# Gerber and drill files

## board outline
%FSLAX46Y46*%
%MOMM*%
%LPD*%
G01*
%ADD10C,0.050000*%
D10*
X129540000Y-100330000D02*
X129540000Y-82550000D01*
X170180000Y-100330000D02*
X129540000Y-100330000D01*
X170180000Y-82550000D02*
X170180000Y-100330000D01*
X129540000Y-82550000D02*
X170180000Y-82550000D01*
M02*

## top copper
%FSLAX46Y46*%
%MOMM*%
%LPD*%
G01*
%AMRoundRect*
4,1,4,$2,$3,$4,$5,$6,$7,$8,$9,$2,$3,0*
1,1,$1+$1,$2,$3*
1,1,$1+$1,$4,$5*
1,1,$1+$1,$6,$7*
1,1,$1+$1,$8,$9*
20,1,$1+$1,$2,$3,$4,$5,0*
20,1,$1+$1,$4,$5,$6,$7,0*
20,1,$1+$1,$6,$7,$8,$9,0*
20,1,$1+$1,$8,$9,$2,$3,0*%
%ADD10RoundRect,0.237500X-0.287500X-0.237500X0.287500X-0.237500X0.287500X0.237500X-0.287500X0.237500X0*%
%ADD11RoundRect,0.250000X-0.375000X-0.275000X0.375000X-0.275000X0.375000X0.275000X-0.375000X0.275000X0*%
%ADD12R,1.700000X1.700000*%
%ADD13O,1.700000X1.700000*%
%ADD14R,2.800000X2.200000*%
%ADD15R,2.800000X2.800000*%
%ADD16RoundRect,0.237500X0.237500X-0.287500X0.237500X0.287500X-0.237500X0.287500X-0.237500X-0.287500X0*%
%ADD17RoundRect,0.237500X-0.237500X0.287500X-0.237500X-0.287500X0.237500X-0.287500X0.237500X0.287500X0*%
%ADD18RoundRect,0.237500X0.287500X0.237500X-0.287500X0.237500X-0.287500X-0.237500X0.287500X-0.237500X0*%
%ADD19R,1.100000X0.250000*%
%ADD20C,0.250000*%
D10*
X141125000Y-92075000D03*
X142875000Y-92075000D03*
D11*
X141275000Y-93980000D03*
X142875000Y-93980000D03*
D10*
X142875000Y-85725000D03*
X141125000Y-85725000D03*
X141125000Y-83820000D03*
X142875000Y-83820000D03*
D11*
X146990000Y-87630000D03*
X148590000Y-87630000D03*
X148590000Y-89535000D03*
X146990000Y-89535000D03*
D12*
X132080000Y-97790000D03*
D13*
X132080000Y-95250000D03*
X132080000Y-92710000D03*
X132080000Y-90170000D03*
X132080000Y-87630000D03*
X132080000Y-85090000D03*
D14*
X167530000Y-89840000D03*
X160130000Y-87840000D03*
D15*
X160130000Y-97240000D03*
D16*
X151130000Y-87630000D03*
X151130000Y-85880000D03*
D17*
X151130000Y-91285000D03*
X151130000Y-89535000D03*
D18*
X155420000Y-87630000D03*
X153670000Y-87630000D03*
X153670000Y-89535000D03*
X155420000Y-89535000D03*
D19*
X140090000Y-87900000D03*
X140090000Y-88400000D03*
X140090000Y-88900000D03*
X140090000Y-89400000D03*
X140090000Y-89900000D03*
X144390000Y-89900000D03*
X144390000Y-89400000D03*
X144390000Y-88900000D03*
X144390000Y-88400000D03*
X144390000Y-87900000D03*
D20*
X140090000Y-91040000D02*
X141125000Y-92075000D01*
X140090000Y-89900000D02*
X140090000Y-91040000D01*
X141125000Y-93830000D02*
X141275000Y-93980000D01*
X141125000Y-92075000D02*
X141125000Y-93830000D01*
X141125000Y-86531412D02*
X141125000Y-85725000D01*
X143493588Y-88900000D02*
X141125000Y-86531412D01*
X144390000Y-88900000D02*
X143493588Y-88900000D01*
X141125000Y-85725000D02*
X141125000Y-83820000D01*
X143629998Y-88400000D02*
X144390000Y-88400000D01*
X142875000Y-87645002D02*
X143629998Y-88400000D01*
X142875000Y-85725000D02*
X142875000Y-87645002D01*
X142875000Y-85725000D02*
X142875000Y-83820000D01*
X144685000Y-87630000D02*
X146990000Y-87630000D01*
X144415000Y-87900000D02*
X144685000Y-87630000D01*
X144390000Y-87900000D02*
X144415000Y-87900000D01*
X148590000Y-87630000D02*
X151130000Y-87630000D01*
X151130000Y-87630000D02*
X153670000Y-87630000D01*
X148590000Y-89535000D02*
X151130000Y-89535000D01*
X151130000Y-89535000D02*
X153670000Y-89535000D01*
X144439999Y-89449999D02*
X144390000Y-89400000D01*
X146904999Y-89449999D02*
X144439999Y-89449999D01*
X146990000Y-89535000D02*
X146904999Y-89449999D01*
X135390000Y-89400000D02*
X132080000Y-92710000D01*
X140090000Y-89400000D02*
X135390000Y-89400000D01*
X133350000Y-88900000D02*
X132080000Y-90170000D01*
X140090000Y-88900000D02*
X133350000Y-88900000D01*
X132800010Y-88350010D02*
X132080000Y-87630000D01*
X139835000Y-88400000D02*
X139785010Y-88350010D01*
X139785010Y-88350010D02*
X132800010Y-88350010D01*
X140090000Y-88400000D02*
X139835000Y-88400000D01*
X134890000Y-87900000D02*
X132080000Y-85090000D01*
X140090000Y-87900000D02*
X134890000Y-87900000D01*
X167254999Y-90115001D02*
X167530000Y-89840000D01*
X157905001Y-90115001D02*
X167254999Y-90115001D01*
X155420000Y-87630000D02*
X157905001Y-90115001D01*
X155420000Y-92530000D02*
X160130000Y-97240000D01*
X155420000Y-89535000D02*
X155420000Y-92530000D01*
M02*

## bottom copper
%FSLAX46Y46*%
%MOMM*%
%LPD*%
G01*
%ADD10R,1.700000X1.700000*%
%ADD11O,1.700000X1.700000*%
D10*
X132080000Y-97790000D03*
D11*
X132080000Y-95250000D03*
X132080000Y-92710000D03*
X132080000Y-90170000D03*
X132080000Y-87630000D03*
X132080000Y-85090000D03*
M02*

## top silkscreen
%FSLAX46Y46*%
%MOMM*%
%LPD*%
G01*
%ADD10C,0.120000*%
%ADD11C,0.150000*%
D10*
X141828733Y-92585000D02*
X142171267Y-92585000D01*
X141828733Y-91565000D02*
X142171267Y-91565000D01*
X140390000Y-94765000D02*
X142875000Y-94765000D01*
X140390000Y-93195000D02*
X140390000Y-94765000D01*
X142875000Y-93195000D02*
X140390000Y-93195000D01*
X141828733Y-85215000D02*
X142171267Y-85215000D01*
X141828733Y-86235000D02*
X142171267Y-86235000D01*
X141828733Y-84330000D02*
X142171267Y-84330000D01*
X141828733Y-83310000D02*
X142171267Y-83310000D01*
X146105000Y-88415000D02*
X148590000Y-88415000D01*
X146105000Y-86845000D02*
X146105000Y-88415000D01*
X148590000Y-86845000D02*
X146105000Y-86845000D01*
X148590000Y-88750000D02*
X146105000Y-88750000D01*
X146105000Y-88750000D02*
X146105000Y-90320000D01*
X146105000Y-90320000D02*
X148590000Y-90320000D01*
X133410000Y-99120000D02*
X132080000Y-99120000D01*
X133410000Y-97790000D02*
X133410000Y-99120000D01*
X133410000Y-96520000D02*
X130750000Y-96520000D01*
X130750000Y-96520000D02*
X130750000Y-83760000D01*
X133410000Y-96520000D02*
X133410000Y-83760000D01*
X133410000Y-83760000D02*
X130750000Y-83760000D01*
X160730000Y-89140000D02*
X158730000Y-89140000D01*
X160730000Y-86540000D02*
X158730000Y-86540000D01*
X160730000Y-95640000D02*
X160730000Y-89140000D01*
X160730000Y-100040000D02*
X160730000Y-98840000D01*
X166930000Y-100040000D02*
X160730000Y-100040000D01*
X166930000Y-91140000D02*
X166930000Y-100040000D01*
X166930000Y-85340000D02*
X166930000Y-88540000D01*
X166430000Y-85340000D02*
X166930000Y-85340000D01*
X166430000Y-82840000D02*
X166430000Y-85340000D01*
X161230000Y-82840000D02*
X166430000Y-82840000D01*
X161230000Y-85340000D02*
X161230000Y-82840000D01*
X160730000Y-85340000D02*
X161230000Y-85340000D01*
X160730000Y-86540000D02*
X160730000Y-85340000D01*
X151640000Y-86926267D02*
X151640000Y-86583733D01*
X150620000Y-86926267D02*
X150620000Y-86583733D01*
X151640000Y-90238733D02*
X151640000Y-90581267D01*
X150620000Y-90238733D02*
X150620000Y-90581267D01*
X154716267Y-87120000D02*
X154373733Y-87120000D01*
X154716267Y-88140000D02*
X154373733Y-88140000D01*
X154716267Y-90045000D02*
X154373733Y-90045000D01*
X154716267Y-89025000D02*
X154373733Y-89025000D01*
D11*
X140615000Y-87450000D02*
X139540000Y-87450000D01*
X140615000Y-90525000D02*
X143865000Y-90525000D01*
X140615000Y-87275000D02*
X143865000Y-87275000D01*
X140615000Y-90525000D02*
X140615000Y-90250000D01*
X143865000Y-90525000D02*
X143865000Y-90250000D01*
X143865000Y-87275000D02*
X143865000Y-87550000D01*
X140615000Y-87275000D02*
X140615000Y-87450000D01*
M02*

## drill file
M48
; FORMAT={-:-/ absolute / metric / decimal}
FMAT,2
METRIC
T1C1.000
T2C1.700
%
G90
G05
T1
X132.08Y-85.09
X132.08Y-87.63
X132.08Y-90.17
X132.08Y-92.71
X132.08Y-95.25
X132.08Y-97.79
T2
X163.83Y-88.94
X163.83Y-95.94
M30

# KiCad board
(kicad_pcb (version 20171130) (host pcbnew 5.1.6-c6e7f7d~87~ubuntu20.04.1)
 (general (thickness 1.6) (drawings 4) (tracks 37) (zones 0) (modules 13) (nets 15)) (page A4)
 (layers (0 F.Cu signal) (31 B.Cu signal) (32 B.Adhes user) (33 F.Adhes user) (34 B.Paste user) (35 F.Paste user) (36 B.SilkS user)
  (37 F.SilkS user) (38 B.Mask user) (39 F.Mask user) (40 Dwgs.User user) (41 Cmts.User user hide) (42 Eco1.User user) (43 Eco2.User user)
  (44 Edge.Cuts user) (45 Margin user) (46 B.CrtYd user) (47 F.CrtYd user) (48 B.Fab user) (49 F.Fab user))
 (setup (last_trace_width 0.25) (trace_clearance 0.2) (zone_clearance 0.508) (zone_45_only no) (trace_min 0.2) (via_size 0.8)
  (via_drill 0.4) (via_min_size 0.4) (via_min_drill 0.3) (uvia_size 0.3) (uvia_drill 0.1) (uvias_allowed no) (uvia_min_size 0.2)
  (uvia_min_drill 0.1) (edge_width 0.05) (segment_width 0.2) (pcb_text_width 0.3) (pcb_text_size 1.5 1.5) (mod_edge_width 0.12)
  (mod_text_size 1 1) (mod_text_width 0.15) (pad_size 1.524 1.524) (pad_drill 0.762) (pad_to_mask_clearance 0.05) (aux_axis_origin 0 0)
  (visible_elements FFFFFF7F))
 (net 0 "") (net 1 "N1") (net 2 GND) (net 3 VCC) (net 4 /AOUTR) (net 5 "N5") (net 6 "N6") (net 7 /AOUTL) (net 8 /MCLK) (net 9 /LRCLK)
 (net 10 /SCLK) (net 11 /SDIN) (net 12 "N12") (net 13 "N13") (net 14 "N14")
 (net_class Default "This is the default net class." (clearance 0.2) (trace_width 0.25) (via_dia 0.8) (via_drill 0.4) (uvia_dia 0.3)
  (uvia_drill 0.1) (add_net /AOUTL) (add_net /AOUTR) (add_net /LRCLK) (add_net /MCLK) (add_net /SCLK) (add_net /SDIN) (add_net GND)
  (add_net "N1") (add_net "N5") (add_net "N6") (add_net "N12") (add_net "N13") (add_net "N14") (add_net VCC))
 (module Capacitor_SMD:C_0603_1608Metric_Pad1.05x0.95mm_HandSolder (layer F.Cu) (at 142 92.075)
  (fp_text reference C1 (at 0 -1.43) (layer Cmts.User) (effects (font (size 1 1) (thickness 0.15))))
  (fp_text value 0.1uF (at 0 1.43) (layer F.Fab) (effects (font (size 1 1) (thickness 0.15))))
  (fp_line (start -0.171267 0.51) (end 0.171267 0.51) (layer F.SilkS) (width 0.12))
  (fp_line (start -0.171267 -0.51) (end 0.171267 -0.51) (layer F.SilkS) (width 0.12))
  (pad 1 smd roundrect (at -0.875 0) (size 1.05 0.95) (layers F.Cu F.Paste F.Mask) (roundrect_rratio 0.25) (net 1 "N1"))
  (pad 2 smd roundrect (at 0.875 0) (size 1.05 0.95) (layers F.Cu F.Paste F.Mask) (roundrect_rratio 0.25) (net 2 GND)))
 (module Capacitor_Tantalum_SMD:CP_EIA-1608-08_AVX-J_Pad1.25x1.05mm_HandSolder (layer F.Cu) (at 142.075 93.98)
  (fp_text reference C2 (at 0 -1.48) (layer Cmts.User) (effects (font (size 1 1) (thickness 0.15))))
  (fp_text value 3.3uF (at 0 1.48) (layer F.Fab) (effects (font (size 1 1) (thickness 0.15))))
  (fp_line (start -1.685 0.785) (end 0.8 0.785) (layer F.SilkS) (width 0.12))
  (fp_line (start -1.685 -0.785) (end -1.685 0.785) (layer F.SilkS) (width 0.12))
  (fp_line (start 0.8 -0.785) (end -1.685 -0.785) (layer F.SilkS) (width 0.12))
  (pad 1 smd roundrect (at -0.8 0) (size 1.25 1.05) (layers F.Cu F.Paste F.Mask) (roundrect_rratio 0.238095) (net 1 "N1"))
  (pad 2 smd roundrect (at 0.8 0) (size 1.25 1.05) (layers F.Cu F.Paste F.Mask) (roundrect_rratio 0.238095) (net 2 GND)))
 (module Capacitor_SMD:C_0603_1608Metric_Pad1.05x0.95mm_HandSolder (layer F.Cu) (at 142 85.725)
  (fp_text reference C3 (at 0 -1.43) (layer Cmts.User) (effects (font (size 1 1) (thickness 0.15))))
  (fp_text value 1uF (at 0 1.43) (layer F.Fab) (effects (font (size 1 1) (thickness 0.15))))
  (fp_line (start -0.171267 -0.51) (end 0.171267 -0.51) (layer F.SilkS) (width 0.12))
  (fp_line (start -0.171267 0.51) (end 0.171267 0.51) (layer F.SilkS) (width 0.12))
  (pad 2 smd roundrect (at 0.875 0) (size 1.05 0.95) (layers F.Cu F.Paste F.Mask) (roundrect_rratio 0.25) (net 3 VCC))
  (pad 1 smd roundrect (at -0.875 0) (size 1.05 0.95) (layers F.Cu F.Paste F.Mask) (roundrect_rratio 0.25) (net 2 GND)))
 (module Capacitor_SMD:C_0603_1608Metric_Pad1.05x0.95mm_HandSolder (layer F.Cu) (at 142 83.82)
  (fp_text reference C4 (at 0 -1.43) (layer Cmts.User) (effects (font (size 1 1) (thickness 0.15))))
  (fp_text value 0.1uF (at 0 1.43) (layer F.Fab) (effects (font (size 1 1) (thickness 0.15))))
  (fp_line (start -0.171267 0.51) (end 0.171267 0.51) (layer F.SilkS) (width 0.12))
  (fp_line (start -0.171267 -0.51) (end 0.171267 -0.51) (layer F.SilkS) (width 0.12))
  (pad 1 smd roundrect (at -0.875 0) (size 1.05 0.95) (layers F.Cu F.Paste F.Mask) (roundrect_rratio 0.25) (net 2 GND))
  (pad 2 smd roundrect (at 0.875 0) (size 1.05 0.95) (layers F.Cu F.Paste F.Mask) (roundrect_rratio 0.25) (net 3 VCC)))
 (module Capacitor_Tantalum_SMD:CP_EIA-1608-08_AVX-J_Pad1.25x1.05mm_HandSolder (layer F.Cu) (at 147.79 87.63)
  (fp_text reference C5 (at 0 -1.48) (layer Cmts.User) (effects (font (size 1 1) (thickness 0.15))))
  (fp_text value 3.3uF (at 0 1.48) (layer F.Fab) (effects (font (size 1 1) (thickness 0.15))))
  (fp_line (start -1.685 0.785) (end 0.8 0.785) (layer F.SilkS) (width 0.12))
  (fp_line (start -1.685 -0.785) (end -1.685 0.785) (layer F.SilkS) (width 0.12))
  (fp_line (start 0.8 -0.785) (end -1.685 -0.785) (layer F.SilkS) (width 0.12))
  (pad 1 smd roundrect (at -0.8 0) (size 1.25 1.05) (layers F.Cu F.Paste F.Mask) (roundrect_rratio 0.238095) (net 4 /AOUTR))
  (pad 2 smd roundrect (at 0.8 0) (size 1.25 1.05) (layers F.Cu F.Paste F.Mask) (roundrect_rratio 0.238095) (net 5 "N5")))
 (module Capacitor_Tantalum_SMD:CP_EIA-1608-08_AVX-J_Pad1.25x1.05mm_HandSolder (layer F.Cu) (at 147.79 89.535)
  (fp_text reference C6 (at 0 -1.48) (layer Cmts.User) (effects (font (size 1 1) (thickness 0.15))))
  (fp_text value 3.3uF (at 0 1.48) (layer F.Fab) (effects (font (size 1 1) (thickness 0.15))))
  (fp_line (start 0.8 -0.785) (end -1.685 -0.785) (layer F.SilkS) (width 0.12))
  (fp_line (start -1.685 -0.785) (end -1.685 0.785) (layer F.SilkS) (width 0.12))
  (fp_line (start -1.685 0.785) (end 0.8 0.785) (layer F.SilkS) (width 0.12))
  (pad 2 smd roundrect (at 0.8 0) (size 1.25 1.05) (layers F.Cu F.Paste F.Mask) (roundrect_rratio 0.238095) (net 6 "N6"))
  (pad 1 smd roundrect (at -0.8 0) (size 1.25 1.05) (layers F.Cu F.Paste F.Mask) (roundrect_rratio 0.238095) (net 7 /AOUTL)))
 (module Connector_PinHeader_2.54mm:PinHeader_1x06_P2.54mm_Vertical (layer F.Cu) (at 132.08 97.79 180)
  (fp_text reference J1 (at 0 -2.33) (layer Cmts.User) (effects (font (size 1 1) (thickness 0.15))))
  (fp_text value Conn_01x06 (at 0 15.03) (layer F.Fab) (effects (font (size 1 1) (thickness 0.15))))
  (fp_line (start -1.33 -1.33) (end 0 -1.33) (layer F.SilkS) (width 0.12))
  (fp_line (start -1.33 0) (end -1.33 -1.33) (layer F.SilkS) (width 0.12))
  (fp_line (start -1.33 1.27) (end 1.33 1.27) (layer F.SilkS) (width 0.12))
  (fp_line (start 1.33 1.27) (end 1.33 14.03) (layer F.SilkS) (width 0.12))
  (fp_line (start -1.33 1.27) (end -1.33 14.03) (layer F.SilkS) (width 0.12))
  (fp_line (start -1.33 14.03) (end 1.33 14.03) (layer F.SilkS) (width 0.12))
  (pad 1 thru_hole rect (at 0 0 180) (size 1.7 1.7) (drill 1) (layers *.Cu *.Mask) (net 3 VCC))
  (pad 2 thru_hole oval (at 0 2.54 180) (size 1.7 1.7) (drill 1) (layers *.Cu *.Mask) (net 2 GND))
  (pad 3 thru_hole oval (at 0 5.08 180) (size 1.7 1.7) (drill 1) (layers *.Cu *.Mask) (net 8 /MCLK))
  (pad 4 thru_hole oval (at 0 7.62 180) (size 1.7 1.7) (drill 1) (layers *.Cu *.Mask) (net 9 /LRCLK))
  (pad 5 thru_hole oval (at 0 10.16 180) (size 1.7 1.7) (drill 1) (layers *.Cu *.Mask) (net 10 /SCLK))
  (pad 6 thru_hole oval (at 0 12.7 180) (size 1.7 1.7) (drill 1) (layers *.Cu *.Mask) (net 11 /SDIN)))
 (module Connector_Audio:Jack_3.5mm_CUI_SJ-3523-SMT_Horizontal (layer F.Cu) (at 163.83 91.44)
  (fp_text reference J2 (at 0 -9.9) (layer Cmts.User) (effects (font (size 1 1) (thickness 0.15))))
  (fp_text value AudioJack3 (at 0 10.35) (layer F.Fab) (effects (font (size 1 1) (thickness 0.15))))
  (fp_line (start -3.1 -2.3) (end -5.1 -2.3) (layer F.SilkS) (width 0.12))
  (fp_line (start -3.1 -4.9) (end -5.1 -4.9) (layer F.SilkS) (width 0.12))
  (fp_line (start -3.1 4.2) (end -3.1 -2.3) (layer F.SilkS) (width 0.12))
  (fp_line (start -3.1 8.6) (end -3.1 7.4) (layer F.SilkS) (width 0.12))
  (fp_line (start 3.1 8.6) (end -3.1 8.6) (layer F.SilkS) (width 0.12))
  (fp_line (start 3.1 -0.3) (end 3.1 8.6) (layer F.SilkS) (width 0.12))
  (fp_line (start 3.1 -6.1) (end 3.1 -2.9) (layer F.SilkS) (width 0.12))
  (fp_line (start 2.6 -6.1) (end 3.1 -6.1) (layer F.SilkS) (width 0.12))
  (fp_line (start 2.6 -8.6) (end 2.6 -6.1) (layer F.SilkS) (width 0.12))
  (fp_line (start -2.6 -8.6) (end 2.6 -8.6) (layer F.SilkS) (width 0.12))
  (fp_line (start -2.6 -6.1) (end -2.6 -8.6) (layer F.SilkS) (width 0.12))
  (fp_line (start -3.1 -6.1) (end -2.6 -6.1) (layer F.SilkS) (width 0.12))
  (fp_line (start -3.1 -4.9) (end -3.1 -6.1) (layer F.SilkS) (width 0.12))
  (pad R smd rect (at 3.7 -1.6) (size 2.8 2.2) (layers F.Cu F.Paste F.Mask) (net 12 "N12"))
  (pad S smd rect (at -3.7 -3.6) (size 2.8 2.2) (layers F.Cu F.Paste F.Mask) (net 2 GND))
  (pad T smd rect (at -3.7 5.8) (size 2.8 2.8) (layers F.Cu F.Paste F.Mask) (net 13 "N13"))
  (pad "" np_thru_hole circle (at 0 -2.5) (size 1.7 1.7) (drill 1.7) (layers *.Cu *.Mask))
  (pad "" np_thru_hole circle (at 0 4.5) (size 1.7 1.7) (drill 1.7) (layers *.Cu *.Mask)))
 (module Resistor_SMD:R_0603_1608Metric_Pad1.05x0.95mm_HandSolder (layer F.Cu) (at 151.13 86.755 90)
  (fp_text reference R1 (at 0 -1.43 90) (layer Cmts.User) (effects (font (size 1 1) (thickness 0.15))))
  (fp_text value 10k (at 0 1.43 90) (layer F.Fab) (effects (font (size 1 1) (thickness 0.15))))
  (fp_line (start -0.171267 0.51) (end 0.171267 0.51) (layer F.SilkS) (width 0.12))
  (fp_line (start -0.171267 -0.51) (end 0.171267 -0.51) (layer F.SilkS) (width 0.12))
  (pad 1 smd roundrect (at -0.875 0 90) (size 1.05 0.95) (layers F.Cu F.Paste F.Mask) (roundrect_rratio 0.25) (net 5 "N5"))
  (pad 2 smd roundrect (at 0.875 0 90) (size 1.05 0.95) (layers F.Cu F.Paste F.Mask) (roundrect_rratio 0.25) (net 2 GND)))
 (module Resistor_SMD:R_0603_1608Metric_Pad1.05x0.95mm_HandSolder (layer F.Cu) (at 151.13 90.41 270)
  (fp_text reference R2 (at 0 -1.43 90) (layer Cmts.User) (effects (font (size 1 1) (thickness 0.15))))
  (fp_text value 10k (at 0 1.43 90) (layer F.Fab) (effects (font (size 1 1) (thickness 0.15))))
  (fp_line (start -0.171267 -0.51) (end 0.171267 -0.51) (layer F.SilkS) (width 0.12))
  (fp_line (start -0.171267 0.51) (end 0.171267 0.51) (layer F.SilkS) (width 0.12))
  (pad 2 smd roundrect (at 0.875 0 270) (size 1.05 0.95) (layers F.Cu F.Paste F.Mask) (roundrect_rratio 0.25) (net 2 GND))
  (pad 1 smd roundrect (at -0.875 0 270) (size 1.05 0.95) (layers F.Cu F.Paste F.Mask) (roundrect_rratio 0.25) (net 6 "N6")))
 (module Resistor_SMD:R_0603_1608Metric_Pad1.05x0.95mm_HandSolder (layer F.Cu) (at 154.545 87.63 180)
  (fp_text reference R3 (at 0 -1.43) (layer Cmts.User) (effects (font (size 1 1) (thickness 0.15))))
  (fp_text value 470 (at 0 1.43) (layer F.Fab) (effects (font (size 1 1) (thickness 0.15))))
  (fp_line (start -0.171267 0.51) (end 0.171267 0.51) (layer F.SilkS) (width 0.12))
  (fp_line (start -0.171267 -0.51) (end 0.171267 -0.51) (layer F.SilkS) (width 0.12))
  (pad 1 smd roundrect (at -0.875 0 180) (size 1.05 0.95) (layers F.Cu F.Paste F.Mask) (roundrect_rratio 0.25) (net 12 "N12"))
  (pad 2 smd roundrect (at 0.875 0 180) (size 1.05 0.95) (layers F.Cu F.Paste F.Mask) (roundrect_rratio 0.25) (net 5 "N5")))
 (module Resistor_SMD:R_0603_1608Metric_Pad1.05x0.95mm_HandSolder (layer F.Cu) (at 154.545 89.535 180)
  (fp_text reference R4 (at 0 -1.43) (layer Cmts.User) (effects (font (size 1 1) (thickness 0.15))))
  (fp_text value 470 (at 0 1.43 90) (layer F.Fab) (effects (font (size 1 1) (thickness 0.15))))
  (fp_line (start -0.171267 -0.51) (end 0.171267 -0.51) (layer F.SilkS) (width 0.12))
  (fp_line (start -0.171267 0.51) (end 0.171267 0.51) (layer F.SilkS) (width 0.12))
  (pad 2 smd roundrect (at 0.875 0 180) (size 1.05 0.95) (layers F.Cu F.Paste F.Mask) (roundrect_rratio 0.25) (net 6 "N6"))
  (pad 1 smd roundrect (at -0.875 0 180) (size 1.05 0.95) (layers F.Cu F.Paste F.Mask) (roundrect_rratio 0.25) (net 13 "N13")))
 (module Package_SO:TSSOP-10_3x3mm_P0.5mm (layer F.Cu) (at 142.24 88.9)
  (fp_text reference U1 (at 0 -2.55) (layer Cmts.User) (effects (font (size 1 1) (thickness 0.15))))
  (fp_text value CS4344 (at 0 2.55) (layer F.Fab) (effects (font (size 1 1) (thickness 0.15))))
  (fp_line (start -1.625 -1.45) (end -2.7 -1.45) (layer F.SilkS) (width 0.15))
  (fp_line (start -1.625 1.625) (end 1.625 1.625) (layer F.SilkS) (width 0.15))
  (fp_line (start -1.625 -1.625) (end 1.625 -1.625) (layer F.SilkS) (width 0.15))
  (fp_line (start -1.625 1.625) (end -1.625 1.35) (layer F.SilkS) (width 0.15))
  (fp_line (start 1.625 1.625) (end 1.625 1.35) (layer F.SilkS) (width 0.15))
  (fp_line (start 1.625 -1.625) (end 1.625 -1.35) (layer F.SilkS) (width 0.15))
  (fp_line (start -1.625 -1.625) (end -1.625 -1.45) (layer F.SilkS) (width 0.15))
  (pad 1 smd rect (at -2.15 -1) (size 1.1 0.25) (layers F.Cu F.Paste F.Mask) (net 11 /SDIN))
  (pad 2 smd rect (at -2.15 -0.5) (size 1.1 0.25) (layers F.Cu F.Paste F.Mask) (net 10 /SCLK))
  (pad 3 smd rect (at -2.15 0) (size 1.1 0.25) (layers F.Cu F.Paste F.Mask) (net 9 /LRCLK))
  (pad 4 smd rect (at -2.15 0.5) (size 1.1 0.25) (layers F.Cu F.Paste F.Mask) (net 8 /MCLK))
  (pad 5 smd rect (at -2.15 1) (size 1.1 0.25) (layers F.Cu F.Paste F.Mask) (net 1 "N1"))
  (pad 6 smd rect (at 2.15 1) (size 1.1 0.25) (layers F.Cu F.Paste F.Mask) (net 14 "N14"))
  (pad 7 smd rect (at 2.15 0.5) (size 1.1 0.25) (layers F.Cu F.Paste F.Mask) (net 7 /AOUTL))
  (pad 8 smd rect (at 2.15 0) (size 1.1 0.25) (layers F.Cu F.Paste F.Mask) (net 2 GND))
  (pad 9 smd rect (at 2.15 -0.5) (size 1.1 0.25) (layers F.Cu F.Paste F.Mask) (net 3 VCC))
  (pad 10 smd rect (at 2.15 -1) (size 1.1 0.25) (layers F.Cu F.Paste F.Mask) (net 4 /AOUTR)))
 (gr_line (start 129.54 100.33) (end 129.54 82.55) (layer Edge.Cuts) (width 0.05))
 (gr_line (start 170.18 100.33) (end 129.54 100.33) (layer Edge.Cuts) (width 0.05))
 (gr_line (start 170.18 82.55) (end 170.18 100.33) (layer Edge.Cuts) (width 0.05))
 (gr_line (start 129.54 82.55) (end 170.18 82.55) (layer Edge.Cuts) (width 0.05))
 (segment (start 140.09 91.04) (end 141.125 92.075) (width 0.25) (layer F.Cu) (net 1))
 (segment (start 140.09 89.9) (end 140.09 91.04) (width 0.25) (layer F.Cu) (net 1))
 (segment (start 141.125 93.83) (end 141.275 93.98) (width 0.25) (layer F.Cu) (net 1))
 (segment (start 141.125 92.075) (end 141.125 93.83) (width 0.25) (layer F.Cu) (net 1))
 (segment (start 141.125 86.531412) (end 141.125 85.725) (width 0.25) (layer F.Cu) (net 2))
 (segment (start 143.493588 88.9) (end 141.125 86.531412) (width 0.25) (layer F.Cu) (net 2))
 (segment (start 144.39 88.9) (end 143.493588 88.9) (width 0.25) (layer F.Cu) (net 2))
 (segment (start 141.125 85.725) (end 141.125 83.82) (width 0.25) (layer F.Cu) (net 2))
 (segment (start 143.629998 88.4) (end 144.39 88.4) (width 0.25) (layer F.Cu) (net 3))
 (segment (start 142.875 87.645002) (end 143.629998 88.4) (width 0.25) (layer F.Cu) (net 3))
 (segment (start 142.875 85.725) (end 142.875 87.645002) (width 0.25) (layer F.Cu) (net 3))
 (segment (start 142.875 85.725) (end 142.875 83.82) (width 0.25) (layer F.Cu) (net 3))
 (segment (start 144.685 87.63) (end 146.99 87.63) (width 0.25) (layer F.Cu) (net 4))
 (segment (start 144.415 87.9) (end 144.685 87.63) (width 0.25) (layer F.Cu) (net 4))
 (segment (start 144.39 87.9) (end 144.415 87.9) (width 0.25) (layer F.Cu) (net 4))
 (segment (start 148.59 87.63) (end 151.13 87.63) (width 0.25) (layer F.Cu) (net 5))
 (segment (start 151.13 87.63) (end 153.67 87.63) (width 0.25) (layer F.Cu) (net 5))
 (segment (start 148.59 89.535) (end 151.13 89.535) (width 0.25) (layer F.Cu) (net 6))
 (segment (start 151.13 89.535) (end 153.67 89.535) (width 0.25) (layer F.Cu) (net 6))
 (segment (start 144.439999 89.449999) (end 144.39 89.4) (width 0.25) (layer F.Cu) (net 7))
 (segment (start 146.904999 89.449999) (end 144.439999 89.449999) (width 0.25) (layer F.Cu) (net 7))
 (segment (start 146.99 89.535) (end 146.904999 89.449999) (width 0.25) (layer F.Cu) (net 7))
 (segment (start 135.39 89.4) (end 132.08 92.71) (width 0.25) (layer F.Cu) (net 8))
 (segment (start 140.09 89.4) (end 135.39 89.4) (width 0.25) (layer F.Cu) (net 8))
 (segment (start 133.35 88.9) (end 132.08 90.17) (width 0.25) (layer F.Cu) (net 9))
 (segment (start 140.09 88.9) (end 133.35 88.9) (width 0.25) (layer F.Cu) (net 9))
 (segment (start 132.80001 88.35001) (end 132.08 87.63) (width 0.25) (layer F.Cu) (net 10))
 (segment (start 139.835 88.4) (end 139.78501 88.35001) (width 0.25) (layer F.Cu) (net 10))
 (segment (start 139.78501 88.35001) (end 132.80001 88.35001) (width 0.25) (layer F.Cu) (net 10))
 (segment (start 140.09 88.4) (end 139.835 88.4) (width 0.25) (layer F.Cu) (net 10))
 (segment (start 134.89 87.9) (end 132.08 85.09) (width 0.25) (layer F.Cu) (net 11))
 (segment (start 140.09 87.9) (end 134.89 87.9) (width 0.25) (layer F.Cu) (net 11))
 (segment (start 167.254999 90.115001) (end 167.53 89.84) (width 0.25) (layer F.Cu) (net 12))
 (segment (start 157.905001 90.115001) (end 167.254999 90.115001) (width 0.25) (layer F.Cu) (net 12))
 (segment (start 155.42 87.63) (end 157.905001 90.115001) (width 0.25) (layer F.Cu) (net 12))
 (segment (start 155.42 92.53) (end 160.13 97.24) (width 0.25) (layer F.Cu) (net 13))
 (segment (start 155.42 89.535) (end 155.42 92.53) (width 0.25) (layer F.Cu) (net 13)))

